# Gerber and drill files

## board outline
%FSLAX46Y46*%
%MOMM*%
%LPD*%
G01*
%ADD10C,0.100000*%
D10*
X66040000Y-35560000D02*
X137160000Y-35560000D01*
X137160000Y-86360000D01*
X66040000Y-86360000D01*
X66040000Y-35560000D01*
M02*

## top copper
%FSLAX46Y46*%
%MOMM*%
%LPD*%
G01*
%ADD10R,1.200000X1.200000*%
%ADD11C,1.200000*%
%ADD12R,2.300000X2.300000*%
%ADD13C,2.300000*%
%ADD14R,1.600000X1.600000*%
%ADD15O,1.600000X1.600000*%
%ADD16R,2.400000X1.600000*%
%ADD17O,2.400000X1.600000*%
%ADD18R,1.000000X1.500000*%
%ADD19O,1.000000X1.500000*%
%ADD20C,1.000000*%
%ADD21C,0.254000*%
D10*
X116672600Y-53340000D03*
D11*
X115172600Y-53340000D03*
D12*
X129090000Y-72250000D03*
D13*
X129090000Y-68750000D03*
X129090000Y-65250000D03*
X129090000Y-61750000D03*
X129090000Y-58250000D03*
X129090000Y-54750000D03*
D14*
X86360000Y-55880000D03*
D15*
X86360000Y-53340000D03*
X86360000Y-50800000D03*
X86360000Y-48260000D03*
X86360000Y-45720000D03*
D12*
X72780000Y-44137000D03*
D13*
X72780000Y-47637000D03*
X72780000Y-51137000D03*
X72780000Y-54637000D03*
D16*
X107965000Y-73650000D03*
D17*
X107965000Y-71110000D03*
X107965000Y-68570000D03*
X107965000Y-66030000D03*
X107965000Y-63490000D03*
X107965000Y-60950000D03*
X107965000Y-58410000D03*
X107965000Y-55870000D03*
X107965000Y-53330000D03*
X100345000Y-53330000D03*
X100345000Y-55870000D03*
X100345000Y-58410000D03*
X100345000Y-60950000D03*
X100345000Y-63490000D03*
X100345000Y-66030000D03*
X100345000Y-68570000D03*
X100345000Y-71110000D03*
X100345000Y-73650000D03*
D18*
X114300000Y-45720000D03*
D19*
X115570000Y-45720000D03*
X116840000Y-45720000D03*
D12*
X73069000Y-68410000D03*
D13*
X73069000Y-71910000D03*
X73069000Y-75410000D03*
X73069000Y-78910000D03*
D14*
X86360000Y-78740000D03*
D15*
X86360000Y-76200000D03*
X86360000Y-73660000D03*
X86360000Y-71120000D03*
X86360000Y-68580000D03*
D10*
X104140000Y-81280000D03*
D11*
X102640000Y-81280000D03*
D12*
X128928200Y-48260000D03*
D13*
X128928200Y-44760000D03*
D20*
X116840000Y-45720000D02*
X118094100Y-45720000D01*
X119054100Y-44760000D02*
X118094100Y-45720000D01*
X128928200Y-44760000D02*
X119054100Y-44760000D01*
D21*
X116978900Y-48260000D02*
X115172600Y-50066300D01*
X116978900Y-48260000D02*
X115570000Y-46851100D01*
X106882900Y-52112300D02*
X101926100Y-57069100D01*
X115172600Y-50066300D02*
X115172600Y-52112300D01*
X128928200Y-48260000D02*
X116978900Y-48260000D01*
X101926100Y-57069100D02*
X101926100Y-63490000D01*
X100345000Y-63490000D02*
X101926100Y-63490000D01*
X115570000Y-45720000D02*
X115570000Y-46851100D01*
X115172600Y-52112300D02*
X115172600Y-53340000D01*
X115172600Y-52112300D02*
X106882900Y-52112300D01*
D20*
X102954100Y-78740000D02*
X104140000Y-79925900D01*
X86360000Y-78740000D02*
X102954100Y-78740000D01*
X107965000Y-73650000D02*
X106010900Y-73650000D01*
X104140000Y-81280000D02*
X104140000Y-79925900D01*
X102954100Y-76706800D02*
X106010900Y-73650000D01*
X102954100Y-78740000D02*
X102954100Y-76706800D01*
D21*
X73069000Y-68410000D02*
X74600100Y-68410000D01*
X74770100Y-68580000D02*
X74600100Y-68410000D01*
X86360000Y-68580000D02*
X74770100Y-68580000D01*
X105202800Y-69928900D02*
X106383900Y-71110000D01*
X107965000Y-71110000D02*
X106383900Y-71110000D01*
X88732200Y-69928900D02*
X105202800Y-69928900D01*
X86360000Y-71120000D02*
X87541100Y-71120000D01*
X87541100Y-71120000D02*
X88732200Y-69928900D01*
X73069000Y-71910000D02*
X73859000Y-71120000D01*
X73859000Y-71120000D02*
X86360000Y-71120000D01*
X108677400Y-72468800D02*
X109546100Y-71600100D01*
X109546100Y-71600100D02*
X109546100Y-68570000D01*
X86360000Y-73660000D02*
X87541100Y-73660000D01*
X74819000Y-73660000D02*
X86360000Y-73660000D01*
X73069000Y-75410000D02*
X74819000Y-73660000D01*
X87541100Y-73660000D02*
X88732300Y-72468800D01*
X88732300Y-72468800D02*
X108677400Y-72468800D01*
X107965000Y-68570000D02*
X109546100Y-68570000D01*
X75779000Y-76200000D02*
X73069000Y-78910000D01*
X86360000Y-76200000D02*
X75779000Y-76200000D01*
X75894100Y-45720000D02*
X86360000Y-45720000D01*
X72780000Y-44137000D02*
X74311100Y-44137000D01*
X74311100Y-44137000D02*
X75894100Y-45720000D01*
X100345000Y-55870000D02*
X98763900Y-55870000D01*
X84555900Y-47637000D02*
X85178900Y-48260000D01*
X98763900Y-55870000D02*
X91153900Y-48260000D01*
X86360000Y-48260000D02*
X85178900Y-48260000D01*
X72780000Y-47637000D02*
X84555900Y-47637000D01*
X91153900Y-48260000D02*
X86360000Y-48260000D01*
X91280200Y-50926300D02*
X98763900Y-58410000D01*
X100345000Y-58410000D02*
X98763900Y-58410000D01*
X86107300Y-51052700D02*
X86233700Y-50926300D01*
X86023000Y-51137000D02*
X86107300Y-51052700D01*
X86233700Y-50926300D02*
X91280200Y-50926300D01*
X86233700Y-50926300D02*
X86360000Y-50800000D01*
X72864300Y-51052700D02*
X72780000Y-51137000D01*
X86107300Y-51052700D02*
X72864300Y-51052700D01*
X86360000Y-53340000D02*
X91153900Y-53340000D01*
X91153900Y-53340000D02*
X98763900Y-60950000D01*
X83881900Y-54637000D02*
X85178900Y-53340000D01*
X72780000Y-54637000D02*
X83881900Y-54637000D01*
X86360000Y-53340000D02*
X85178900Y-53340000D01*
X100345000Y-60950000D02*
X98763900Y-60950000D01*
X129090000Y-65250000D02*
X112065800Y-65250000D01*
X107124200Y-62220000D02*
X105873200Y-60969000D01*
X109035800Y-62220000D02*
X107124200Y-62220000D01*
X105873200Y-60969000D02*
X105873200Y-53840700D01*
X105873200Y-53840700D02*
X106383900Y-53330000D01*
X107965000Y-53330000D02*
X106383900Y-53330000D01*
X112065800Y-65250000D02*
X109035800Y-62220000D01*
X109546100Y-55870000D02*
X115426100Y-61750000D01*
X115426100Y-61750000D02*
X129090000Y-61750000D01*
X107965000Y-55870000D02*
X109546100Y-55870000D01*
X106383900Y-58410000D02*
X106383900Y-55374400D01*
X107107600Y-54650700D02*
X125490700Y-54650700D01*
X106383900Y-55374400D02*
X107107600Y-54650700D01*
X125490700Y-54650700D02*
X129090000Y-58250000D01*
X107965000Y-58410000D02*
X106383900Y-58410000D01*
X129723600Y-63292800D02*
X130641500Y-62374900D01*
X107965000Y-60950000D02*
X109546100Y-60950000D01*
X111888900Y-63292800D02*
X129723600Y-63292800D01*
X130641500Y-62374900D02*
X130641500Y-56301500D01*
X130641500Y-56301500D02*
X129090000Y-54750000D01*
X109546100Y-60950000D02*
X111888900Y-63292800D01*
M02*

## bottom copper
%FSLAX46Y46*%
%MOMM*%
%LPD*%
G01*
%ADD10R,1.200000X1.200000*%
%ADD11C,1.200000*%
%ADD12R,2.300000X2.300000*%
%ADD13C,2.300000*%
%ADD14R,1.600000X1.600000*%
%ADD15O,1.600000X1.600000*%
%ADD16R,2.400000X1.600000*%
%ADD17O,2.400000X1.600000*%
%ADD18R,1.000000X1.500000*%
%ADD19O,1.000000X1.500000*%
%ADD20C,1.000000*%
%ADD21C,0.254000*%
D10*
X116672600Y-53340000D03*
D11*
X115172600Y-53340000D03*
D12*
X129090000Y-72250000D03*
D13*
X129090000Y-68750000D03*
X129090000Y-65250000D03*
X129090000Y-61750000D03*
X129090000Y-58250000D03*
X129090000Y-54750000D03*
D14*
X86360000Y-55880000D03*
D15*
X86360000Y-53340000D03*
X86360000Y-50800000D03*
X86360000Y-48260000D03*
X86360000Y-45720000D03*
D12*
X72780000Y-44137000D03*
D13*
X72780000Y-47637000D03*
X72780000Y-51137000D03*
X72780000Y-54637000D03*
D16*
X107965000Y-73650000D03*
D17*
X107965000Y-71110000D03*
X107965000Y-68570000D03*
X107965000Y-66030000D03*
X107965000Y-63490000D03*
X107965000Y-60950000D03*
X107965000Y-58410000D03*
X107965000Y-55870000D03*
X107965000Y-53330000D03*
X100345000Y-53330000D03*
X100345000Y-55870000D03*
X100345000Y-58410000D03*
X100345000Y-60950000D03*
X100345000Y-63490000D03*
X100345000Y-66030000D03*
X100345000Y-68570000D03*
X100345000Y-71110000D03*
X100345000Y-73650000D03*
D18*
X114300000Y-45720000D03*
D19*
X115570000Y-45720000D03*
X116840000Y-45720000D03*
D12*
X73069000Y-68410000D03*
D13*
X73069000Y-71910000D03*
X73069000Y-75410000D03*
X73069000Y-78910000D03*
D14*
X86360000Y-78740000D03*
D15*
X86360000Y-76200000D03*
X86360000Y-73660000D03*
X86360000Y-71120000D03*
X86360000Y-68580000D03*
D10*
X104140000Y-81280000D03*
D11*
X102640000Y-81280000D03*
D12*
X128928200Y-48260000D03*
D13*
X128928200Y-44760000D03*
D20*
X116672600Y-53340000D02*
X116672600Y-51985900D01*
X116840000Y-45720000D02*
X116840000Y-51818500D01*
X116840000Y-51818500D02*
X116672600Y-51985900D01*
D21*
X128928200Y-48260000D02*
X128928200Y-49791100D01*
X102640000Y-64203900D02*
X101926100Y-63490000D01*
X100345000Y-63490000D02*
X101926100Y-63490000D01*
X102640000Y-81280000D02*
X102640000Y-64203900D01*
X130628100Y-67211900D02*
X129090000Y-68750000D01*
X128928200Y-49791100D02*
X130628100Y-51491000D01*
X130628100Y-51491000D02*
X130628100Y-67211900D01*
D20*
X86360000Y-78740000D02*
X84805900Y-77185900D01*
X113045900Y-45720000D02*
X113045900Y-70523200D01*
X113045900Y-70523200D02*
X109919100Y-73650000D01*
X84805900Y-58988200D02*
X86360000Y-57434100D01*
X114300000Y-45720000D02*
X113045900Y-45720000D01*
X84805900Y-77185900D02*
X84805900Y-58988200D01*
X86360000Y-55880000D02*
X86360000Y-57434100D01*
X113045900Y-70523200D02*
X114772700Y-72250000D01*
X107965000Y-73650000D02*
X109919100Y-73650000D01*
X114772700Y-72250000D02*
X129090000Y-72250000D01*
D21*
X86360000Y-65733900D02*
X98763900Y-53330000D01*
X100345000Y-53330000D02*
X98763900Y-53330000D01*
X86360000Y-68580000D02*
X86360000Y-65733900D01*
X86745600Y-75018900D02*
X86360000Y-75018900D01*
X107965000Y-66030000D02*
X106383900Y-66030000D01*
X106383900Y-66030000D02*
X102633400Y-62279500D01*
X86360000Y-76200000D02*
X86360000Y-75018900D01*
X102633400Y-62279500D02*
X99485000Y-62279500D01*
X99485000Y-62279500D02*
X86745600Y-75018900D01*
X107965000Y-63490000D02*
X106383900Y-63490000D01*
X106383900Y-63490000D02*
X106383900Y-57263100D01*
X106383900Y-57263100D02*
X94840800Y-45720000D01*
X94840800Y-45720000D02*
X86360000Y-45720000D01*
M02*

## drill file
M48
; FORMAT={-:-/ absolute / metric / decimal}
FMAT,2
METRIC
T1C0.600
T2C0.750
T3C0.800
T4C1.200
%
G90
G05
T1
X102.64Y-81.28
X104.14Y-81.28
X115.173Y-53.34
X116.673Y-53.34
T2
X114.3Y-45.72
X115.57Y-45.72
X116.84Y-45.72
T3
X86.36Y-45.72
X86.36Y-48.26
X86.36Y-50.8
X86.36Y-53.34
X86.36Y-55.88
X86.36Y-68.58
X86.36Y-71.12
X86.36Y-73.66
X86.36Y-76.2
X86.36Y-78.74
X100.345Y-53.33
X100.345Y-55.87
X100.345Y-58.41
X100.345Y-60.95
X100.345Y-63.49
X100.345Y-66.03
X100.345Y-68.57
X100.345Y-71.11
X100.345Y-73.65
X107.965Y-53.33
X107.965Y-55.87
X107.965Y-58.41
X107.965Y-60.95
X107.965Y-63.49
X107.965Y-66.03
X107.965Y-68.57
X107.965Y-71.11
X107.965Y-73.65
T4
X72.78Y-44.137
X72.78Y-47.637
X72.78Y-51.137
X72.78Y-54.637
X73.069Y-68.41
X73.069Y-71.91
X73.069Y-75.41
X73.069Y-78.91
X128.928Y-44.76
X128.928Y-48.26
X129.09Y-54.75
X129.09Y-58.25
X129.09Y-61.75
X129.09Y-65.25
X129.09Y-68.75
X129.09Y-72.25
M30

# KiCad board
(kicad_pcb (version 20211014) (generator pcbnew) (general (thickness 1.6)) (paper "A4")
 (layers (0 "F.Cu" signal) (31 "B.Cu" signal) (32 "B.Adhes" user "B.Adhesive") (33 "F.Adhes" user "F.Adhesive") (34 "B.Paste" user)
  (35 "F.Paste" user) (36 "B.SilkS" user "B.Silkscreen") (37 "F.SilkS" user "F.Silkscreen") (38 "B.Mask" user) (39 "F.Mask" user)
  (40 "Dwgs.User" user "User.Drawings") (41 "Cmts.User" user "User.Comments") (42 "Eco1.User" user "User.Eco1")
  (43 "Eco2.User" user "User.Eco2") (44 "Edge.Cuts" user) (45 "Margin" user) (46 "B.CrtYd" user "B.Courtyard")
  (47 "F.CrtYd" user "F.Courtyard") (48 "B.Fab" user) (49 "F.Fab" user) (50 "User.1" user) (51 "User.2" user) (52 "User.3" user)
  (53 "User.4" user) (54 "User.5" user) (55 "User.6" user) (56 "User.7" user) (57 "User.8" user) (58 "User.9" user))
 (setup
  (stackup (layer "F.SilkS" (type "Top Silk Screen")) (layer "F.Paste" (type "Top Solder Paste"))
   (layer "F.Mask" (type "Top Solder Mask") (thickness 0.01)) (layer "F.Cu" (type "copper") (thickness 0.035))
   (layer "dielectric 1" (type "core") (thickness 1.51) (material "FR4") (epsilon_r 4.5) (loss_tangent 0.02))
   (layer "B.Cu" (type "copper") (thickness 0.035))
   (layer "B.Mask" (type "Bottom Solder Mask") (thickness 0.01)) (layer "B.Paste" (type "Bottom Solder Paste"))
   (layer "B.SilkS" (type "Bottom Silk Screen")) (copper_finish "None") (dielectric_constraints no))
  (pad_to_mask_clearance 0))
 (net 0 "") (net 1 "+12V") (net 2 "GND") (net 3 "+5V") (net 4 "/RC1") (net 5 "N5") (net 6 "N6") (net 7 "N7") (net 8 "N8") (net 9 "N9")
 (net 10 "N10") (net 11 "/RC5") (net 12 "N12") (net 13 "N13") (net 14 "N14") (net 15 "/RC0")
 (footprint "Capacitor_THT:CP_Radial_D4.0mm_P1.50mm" (layer "F.Cu") (at 116.6726 53.34 180)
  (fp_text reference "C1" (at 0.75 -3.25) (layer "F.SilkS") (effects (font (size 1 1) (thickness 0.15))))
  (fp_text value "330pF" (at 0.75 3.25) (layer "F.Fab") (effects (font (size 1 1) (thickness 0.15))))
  (pad "1" thru_hole rect (at 0 0 180) (size 1.2 1.2) (drill 0.6) (layers *.Cu *.Mask) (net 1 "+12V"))
  (pad "2" thru_hole circle (at 1.5 0 180) (size 1.2 1.2) (drill 0.6) (layers *.Cu *.Mask) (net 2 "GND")))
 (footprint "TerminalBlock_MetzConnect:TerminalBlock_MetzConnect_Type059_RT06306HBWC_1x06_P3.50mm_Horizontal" (layer "F.Cu")
  (at 129.09 72.25 90)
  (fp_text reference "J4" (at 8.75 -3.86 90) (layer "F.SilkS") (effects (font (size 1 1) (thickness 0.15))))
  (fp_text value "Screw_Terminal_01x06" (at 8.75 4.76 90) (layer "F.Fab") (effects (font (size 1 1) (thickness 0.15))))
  (pad "1" thru_hole rect (at 0 0 90) (size 2.3 2.3) (drill 1.2) (layers *.Cu *.Mask) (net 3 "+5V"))
  (pad "2" thru_hole circle (at 3.5 0 90) (size 2.3 2.3) (drill 1.2) (layers *.Cu *.Mask) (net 2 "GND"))
  (pad "3" thru_hole circle (at 7 0 90) (size 2.3 2.3) (drill 1.2) (layers *.Cu *.Mask) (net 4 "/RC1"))
  (pad "4" thru_hole circle (at 10.5 0 90) (size 2.3 2.3) (drill 1.2) (layers *.Cu *.Mask) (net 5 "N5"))
  (pad "5" thru_hole circle (at 14 0 90) (size 2.3 2.3) (drill 1.2) (layers *.Cu *.Mask) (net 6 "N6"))
  (pad "6" thru_hole circle (at 17.5 0 90) (size 2.3 2.3) (drill 1.2) (layers *.Cu *.Mask) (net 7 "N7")))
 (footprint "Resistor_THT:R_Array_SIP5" (layer "F.Cu") (at 86.36 55.88 90)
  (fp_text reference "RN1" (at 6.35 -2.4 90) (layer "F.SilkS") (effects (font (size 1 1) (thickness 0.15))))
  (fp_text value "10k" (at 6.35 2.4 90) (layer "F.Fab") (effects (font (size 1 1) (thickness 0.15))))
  (pad "1" thru_hole rect (at 0 0 90) (size 1.6 1.6) (drill 0.8) (layers *.Cu *.Mask) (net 3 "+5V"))
  (pad "2" thru_hole oval (at 2.54 0 90) (size 1.6 1.6) (drill 0.8) (layers *.Cu *.Mask) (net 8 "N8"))
  (pad "3" thru_hole oval (at 5.08 0 90) (size 1.6 1.6) (drill 0.8) (layers *.Cu *.Mask) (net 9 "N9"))
  (pad "4" thru_hole oval (at 7.62 0 90) (size 1.6 1.6) (drill 0.8) (layers *.Cu *.Mask) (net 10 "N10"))
  (pad "5" thru_hole oval (at 10.16 0 90) (size 1.6 1.6) (drill 0.8) (layers *.Cu *.Mask) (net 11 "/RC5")))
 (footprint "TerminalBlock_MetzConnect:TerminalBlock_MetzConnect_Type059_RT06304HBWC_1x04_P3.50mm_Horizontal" (layer "F.Cu")
  (at 72.78 44.137 -90)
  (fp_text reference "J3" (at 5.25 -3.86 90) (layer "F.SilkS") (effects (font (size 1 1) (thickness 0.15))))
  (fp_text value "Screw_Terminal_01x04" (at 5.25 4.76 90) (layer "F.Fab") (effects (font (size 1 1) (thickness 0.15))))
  (pad "1" thru_hole rect (at 0 0 270) (size 2.3 2.3) (drill 1.2) (layers *.Cu *.Mask) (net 11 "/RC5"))
  (pad "2" thru_hole circle (at 3.5 0 270) (size 2.3 2.3) (drill 1.2) (layers *.Cu *.Mask) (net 10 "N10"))
  (pad "3" thru_hole circle (at 7 0 270) (size 2.3 2.3) (drill 1.2) (layers *.Cu *.Mask) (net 9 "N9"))
  (pad "4" thru_hole circle (at 10.5 0 270) (size 2.3 2.3) (drill 1.2) (layers *.Cu *.Mask) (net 8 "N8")))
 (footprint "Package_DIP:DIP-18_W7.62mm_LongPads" (layer "F.Cu") (at 107.965 73.65 180)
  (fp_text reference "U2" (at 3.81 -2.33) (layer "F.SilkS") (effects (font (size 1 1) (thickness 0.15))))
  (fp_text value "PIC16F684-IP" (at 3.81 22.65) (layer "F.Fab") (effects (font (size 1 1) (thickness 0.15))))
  (pad "1" thru_hole rect (at 0 0 180) (size 2.4 1.6) (drill 0.8) (layers *.Cu *.Mask) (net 3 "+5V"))
  (pad "2" thru_hole oval (at 0 2.54 180) (size 2.4 1.6) (drill 0.8) (layers *.Cu *.Mask) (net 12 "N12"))
  (pad "3" thru_hole oval (at 0 5.08 180) (size 2.4 1.6) (drill 0.8) (layers *.Cu *.Mask) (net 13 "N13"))
  (pad "4" thru_hole oval (at 0 7.62 180) (size 2.4 1.6) (drill 0.8) (layers *.Cu *.Mask) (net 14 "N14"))
  (pad "5" thru_hole oval (at 0 10.16 180) (size 2.4 1.6) (drill 0.8) (layers *.Cu *.Mask) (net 11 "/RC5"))
  (pad "6" thru_hole oval (at 0 12.7 180) (size 2.4 1.6) (drill 0.8) (layers *.Cu *.Mask) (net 7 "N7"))
  (pad "7" thru_hole oval (at 0 15.24 180) (size 2.4 1.6) (drill 0.8) (layers *.Cu *.Mask) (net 6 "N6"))
  (pad "8" thru_hole oval (at 0 17.78 180) (size 2.4 1.6) (drill 0.8) (layers *.Cu *.Mask) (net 5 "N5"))
  (pad "9" thru_hole oval (at 0 20.32 180) (size 2.4 1.6) (drill 0.8) (layers *.Cu *.Mask) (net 4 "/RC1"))
  (pad "10" thru_hole oval (at 7.62 20.32 180) (size 2.4 1.6) (drill 0.8) (layers *.Cu *.Mask) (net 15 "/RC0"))
  (pad "11" thru_hole oval (at 7.62 17.78 180) (size 2.4 1.6) (drill 0.8) (layers *.Cu *.Mask) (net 10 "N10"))
  (pad "12" thru_hole oval (at 7.62 15.24 180) (size 2.4 1.6) (drill 0.8) (layers *.Cu *.Mask) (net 9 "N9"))
  (pad "13" thru_hole oval (at 7.62 12.7 180) (size 2.4 1.6) (drill 0.8) (layers *.Cu *.Mask) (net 8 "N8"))
  (pad "14" thru_hole oval (at 7.62 10.16 180) (size 2.4 1.6) (drill 0.8) (layers *.Cu *.Mask) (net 2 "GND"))
  (pad "15" thru_hole oval (at 7.62 7.62 180) (size 2.4 1.6) (drill 0.8) (layers *.Cu *.Mask))
  (pad "16" thru_hole oval (at 7.62 5.08 180) (size 2.4 1.6) (drill 0.8) (layers *.Cu *.Mask))
  (pad "17" thru_hole oval (at 7.62 2.54 180) (size 2.4 1.6) (drill 0.8) (layers *.Cu *.Mask))
  (pad "18" thru_hole oval (at 7.62 0 180) (size 2.4 1.6) (drill 0.8) (layers *.Cu *.Mask)))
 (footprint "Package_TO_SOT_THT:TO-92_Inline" (layer "F.Cu") (at 114.3 45.72)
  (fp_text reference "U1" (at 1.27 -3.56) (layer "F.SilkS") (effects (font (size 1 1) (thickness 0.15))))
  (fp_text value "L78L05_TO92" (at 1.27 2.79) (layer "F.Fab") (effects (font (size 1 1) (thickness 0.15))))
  (pad "1" thru_hole rect (at 0 0) (size 1 1.5) (drill 0.75) (layers *.Cu *.Mask) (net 3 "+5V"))
  (pad "2" thru_hole oval (at 1.27 0) (size 1 1.5) (drill 0.75) (layers *.Cu *.Mask) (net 2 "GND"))
  (pad "3" thru_hole oval (at 2.54 0) (size 1 1.5) (drill 0.75) (layers *.Cu *.Mask) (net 1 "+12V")))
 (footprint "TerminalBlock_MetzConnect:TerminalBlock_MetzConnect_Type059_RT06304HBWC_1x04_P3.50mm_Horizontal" (layer "F.Cu")
  (at 73.069 68.41 -90)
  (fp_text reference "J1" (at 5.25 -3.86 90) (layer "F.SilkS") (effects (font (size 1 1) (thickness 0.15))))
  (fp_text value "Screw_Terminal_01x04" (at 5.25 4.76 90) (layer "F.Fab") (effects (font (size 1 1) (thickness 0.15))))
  (pad "1" thru_hole rect (at 0 0 270) (size 2.3 2.3) (drill 1.2) (layers *.Cu *.Mask) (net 15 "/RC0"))
  (pad "2" thru_hole circle (at 3.5 0 270) (size 2.3 2.3) (drill 1.2) (layers *.Cu *.Mask) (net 12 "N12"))
  (pad "3" thru_hole circle (at 7 0 270) (size 2.3 2.3) (drill 1.2) (layers *.Cu *.Mask) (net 13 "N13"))
  (pad "4" thru_hole circle (at 10.5 0 270) (size 2.3 2.3) (drill 1.2) (layers *.Cu *.Mask) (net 14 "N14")))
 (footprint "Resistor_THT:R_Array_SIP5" (layer "F.Cu") (at 86.36 78.74 90)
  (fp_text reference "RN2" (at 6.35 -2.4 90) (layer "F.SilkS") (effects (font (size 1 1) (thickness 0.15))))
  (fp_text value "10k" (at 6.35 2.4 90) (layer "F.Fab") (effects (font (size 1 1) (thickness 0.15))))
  (pad "1" thru_hole rect (at 0 0 90) (size 1.6 1.6) (drill 0.8) (layers *.Cu *.Mask) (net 3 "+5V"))
  (pad "2" thru_hole oval (at 2.54 0 90) (size 1.6 1.6) (drill 0.8) (layers *.Cu *.Mask) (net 14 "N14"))
  (pad "3" thru_hole oval (at 5.08 0 90) (size 1.6 1.6) (drill 0.8) (layers *.Cu *.Mask) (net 13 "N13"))
  (pad "4" thru_hole oval (at 7.62 0 90) (size 1.6 1.6) (drill 0.8) (layers *.Cu *.Mask) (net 12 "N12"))
  (pad "5" thru_hole oval (at 10.16 0 90) (size 1.6 1.6) (drill 0.8) (layers *.Cu *.Mask) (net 15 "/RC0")))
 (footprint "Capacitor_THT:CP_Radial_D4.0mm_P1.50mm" (layer "F.Cu") (at 104.14 81.28 180)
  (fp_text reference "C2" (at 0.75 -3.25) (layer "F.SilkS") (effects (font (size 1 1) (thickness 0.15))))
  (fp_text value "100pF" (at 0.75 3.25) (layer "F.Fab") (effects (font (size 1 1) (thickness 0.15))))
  (pad "1" thru_hole rect (at 0 0 180) (size 1.2 1.2) (drill 0.6) (layers *.Cu *.Mask) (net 3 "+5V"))
  (pad "2" thru_hole circle (at 1.5 0 180) (size 1.2 1.2) (drill 0.6) (layers *.Cu *.Mask) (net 2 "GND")))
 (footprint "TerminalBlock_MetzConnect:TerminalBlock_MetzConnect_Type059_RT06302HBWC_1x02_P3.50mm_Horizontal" (layer "F.Cu")
  (at 128.9282 48.26 90)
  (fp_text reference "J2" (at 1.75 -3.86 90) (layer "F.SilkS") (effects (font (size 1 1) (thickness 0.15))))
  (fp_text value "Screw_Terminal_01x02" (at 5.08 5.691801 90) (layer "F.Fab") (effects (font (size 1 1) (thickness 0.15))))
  (pad "1" thru_hole rect (at 0 0 90) (size 2.3 2.3) (drill 1.2) (layers *.Cu *.Mask) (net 2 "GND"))
  (pad "2" thru_hole circle (at 3.5 0 90) (size 2.3 2.3) (drill 1.2) (layers *.Cu *.Mask) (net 1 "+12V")))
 (gr_rect (start 66.04 35.56) (end 137.16 86.36) (layer "Edge.Cuts") (width 0.1) (fill none))
 (segment (start 116.84 45.72) (end 118.0941 45.72) (width 1) (layer "F.Cu") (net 1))
 (segment (start 119.0541 44.76) (end 118.0941 45.72) (width 1) (layer "F.Cu") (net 1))
 (segment (start 128.9282 44.76) (end 119.0541 44.76) (width 1) (layer "F.Cu") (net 1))
 (segment (start 116.6726 53.34) (end 116.6726 51.9859) (width 1) (layer "B.Cu") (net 1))
 (segment (start 116.84 45.72) (end 116.84 51.8185) (width 1) (layer "B.Cu") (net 1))
 (segment (start 116.84 51.8185) (end 116.6726 51.9859) (width 1) (layer "B.Cu") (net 1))
 (segment (start 116.9789 48.26) (end 115.1726 50.0663) (width 0.254) (layer "F.Cu") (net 2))
 (segment (start 116.9789 48.26) (end 115.57 46.8511) (width 0.254) (layer "F.Cu") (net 2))
 (segment (start 106.8829 52.1123) (end 101.9261 57.0691) (width 0.254) (layer "F.Cu") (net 2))
 (segment (start 115.1726 50.0663) (end 115.1726 52.1123) (width 0.254) (layer "F.Cu") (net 2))
 (segment (start 128.9282 48.26) (end 116.9789 48.26) (width 0.254) (layer "F.Cu") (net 2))
 (segment (start 101.9261 57.0691) (end 101.9261 63.49) (width 0.254) (layer "F.Cu") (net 2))
 (segment (start 100.345 63.49) (end 101.9261 63.49) (width 0.254) (layer "F.Cu") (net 2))
 (segment (start 115.57 45.72) (end 115.57 46.8511) (width 0.254) (layer "F.Cu") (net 2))
 (segment (start 115.1726 52.1123) (end 115.1726 53.34) (width 0.254) (layer "F.Cu") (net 2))
 (segment (start 115.1726 52.1123) (end 106.8829 52.1123) (width 0.254) (layer "F.Cu") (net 2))
 (segment (start 128.9282 48.26) (end 128.9282 49.7911) (width 0.254) (layer "B.Cu") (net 2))
 (segment (start 102.64 64.2039) (end 101.9261 63.49) (width 0.254) (layer "B.Cu") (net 2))
 (segment (start 100.345 63.49) (end 101.9261 63.49) (width 0.254) (layer "B.Cu") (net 2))
 (segment (start 102.64 81.28) (end 102.64 64.2039) (width 0.254) (layer "B.Cu") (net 2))
 (segment (start 130.6281 67.2119) (end 129.09 68.75) (width 0.254) (layer "B.Cu") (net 2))
 (segment (start 128.9282 49.7911) (end 130.6281 51.491) (width 0.254) (layer "B.Cu") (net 2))
 (segment (start 130.6281 51.491) (end 130.6281 67.2119) (width 0.254) (layer "B.Cu") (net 2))
 (segment (start 102.9541 78.74) (end 104.14 79.9259) (width 1) (layer "F.Cu") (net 3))
 (segment (start 86.36 78.74) (end 102.9541 78.74) (width 1) (layer "F.Cu") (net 3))
 (segment (start 107.965 73.65) (end 106.0109 73.65) (width 1) (layer "F.Cu") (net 3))
 (segment (start 104.14 81.28) (end 104.14 79.9259) (width 1) (layer "F.Cu") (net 3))
 (segment (start 102.9541 76.7068) (end 106.0109 73.65) (width 1) (layer "F.Cu") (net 3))
 (segment (start 102.9541 78.74) (end 102.9541 76.7068) (width 1) (layer "F.Cu") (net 3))
 (segment (start 86.36 78.74) (end 84.8059 77.1859) (width 1) (layer "B.Cu") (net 3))
 (segment (start 113.0459 45.72) (end 113.0459 70.5232) (width 1) (layer "B.Cu") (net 3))
 (segment (start 113.0459 70.5232) (end 109.9191 73.65) (width 1) (layer "B.Cu") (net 3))
 (segment (start 84.8059 58.9882) (end 86.36 57.4341) (width 1) (layer "B.Cu") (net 3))
 (segment (start 114.3 45.72) (end 113.0459 45.72) (width 1) (layer "B.Cu") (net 3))
 (segment (start 84.8059 77.1859) (end 84.8059 58.9882) (width 1) (layer "B.Cu") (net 3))
 (segment (start 86.36 55.88) (end 86.36 57.4341) (width 1) (layer "B.Cu") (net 3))
 (segment (start 113.0459 70.5232) (end 114.7727 72.25) (width 1) (layer "B.Cu") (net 3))
 (segment (start 107.965 73.65) (end 109.9191 73.65) (width 1) (layer "B.Cu") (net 3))
 (segment (start 114.7727 72.25) (end 129.09 72.25) (width 1) (layer "B.Cu") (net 3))
 (segment (start 73.069 68.41) (end 74.6001 68.41) (width 0.254) (layer "F.Cu") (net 15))
 (segment (start 74.7701 68.58) (end 74.6001 68.41) (width 0.254) (layer "F.Cu") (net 15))
 (segment (start 86.36 68.58) (end 74.7701 68.58) (width 0.254) (layer "F.Cu") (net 15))
 (segment (start 86.36 65.7339) (end 98.7639 53.33) (width 0.254) (layer "B.Cu") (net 15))
 (segment (start 100.345 53.33) (end 98.7639 53.33) (width 0.254) (layer "B.Cu") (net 15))
 (segment (start 86.36 68.58) (end 86.36 65.7339) (width 0.254) (layer "B.Cu") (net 15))
 (segment (start 105.2028 69.9289) (end 106.3839 71.11) (width 0.254) (layer "F.Cu") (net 12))
 (segment (start 107.965 71.11) (end 106.3839 71.11) (width 0.254) (layer "F.Cu") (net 12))
 (segment (start 88.7322 69.9289) (end 105.2028 69.9289) (width 0.254) (layer "F.Cu") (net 12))
 (segment (start 86.36 71.12) (end 87.5411 71.12) (width 0.254) (layer "F.Cu") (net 12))
 (segment (start 87.5411 71.12) (end 88.7322 69.9289) (width 0.254) (layer "F.Cu") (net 12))
 (segment (start 73.069 71.91) (end 73.859 71.12) (width 0.254) (layer "F.Cu") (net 12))
 (segment (start 73.859 71.12) (end 86.36 71.12) (width 0.254) (layer "F.Cu") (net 12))
 (segment (start 108.6774 72.4688) (end 109.5461 71.6001) (width 0.254) (layer "F.Cu") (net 13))
 (segment (start 109.5461 71.6001) (end 109.5461 68.57) (width 0.254) (layer "F.Cu") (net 13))
 (segment (start 86.36 73.66) (end 87.5411 73.66) (width 0.254) (layer "F.Cu") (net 13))
 (segment (start 74.819 73.66) (end 86.36 73.66) (width 0.254) (layer "F.Cu") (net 13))
 (segment (start 73.069 75.41) (end 74.819 73.66) (width 0.254) (layer "F.Cu") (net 13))
 (segment (start 87.5411 73.66) (end 88.7323 72.4688) (width 0.254) (layer "F.Cu") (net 13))
 (segment (start 88.7323 72.4688) (end 108.6774 72.4688) (width 0.254) (layer "F.Cu") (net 13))
 (segment (start 107.965 68.57) (end 109.5461 68.57) (width 0.254) (layer "F.Cu") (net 13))
 (segment (start 75.779 76.2) (end 73.069 78.91) (width 0.254) (layer "F.Cu") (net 14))
 (segment (start 86.36 76.2) (end 75.779 76.2) (width 0.254) (layer "F.Cu") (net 14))
 (segment (start 86.7456 75.0189) (end 86.36 75.0189) (width 0.254) (layer "B.Cu") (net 14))
 (segment (start 107.965 66.03) (end 106.3839 66.03) (width 0.254) (layer "B.Cu") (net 14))
 (segment (start 106.3839 66.03) (end 102.6334 62.2795) (width 0.254) (layer "B.Cu") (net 14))
 (segment (start 86.36 76.2) (end 86.36 75.0189) (width 0.254) (layer "B.Cu") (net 14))
 (segment (start 102.6334 62.2795) (end 99.485 62.2795) (width 0.254) (layer "B.Cu") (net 14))
 (segment (start 99.485 62.2795) (end 86.7456 75.0189) (width 0.254) (layer "B.Cu") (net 14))
 (segment (start 75.8941 45.72) (end 86.36 45.72) (width 0.254) (layer "F.Cu") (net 11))
 (segment (start 72.78 44.137) (end 74.3111 44.137) (width 0.254) (layer "F.Cu") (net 11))
 (segment (start 74.3111 44.137) (end 75.8941 45.72) (width 0.254) (layer "F.Cu") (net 11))
 (segment (start 107.965 63.49) (end 106.3839 63.49) (width 0.254) (layer "B.Cu") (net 11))
 (segment (start 106.3839 63.49) (end 106.3839 57.2631) (width 0.254) (layer "B.Cu") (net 11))
 (segment (start 106.3839 57.2631) (end 94.8408 45.72) (width 0.254) (layer "B.Cu") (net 11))
 (segment (start 94.8408 45.72) (end 86.36 45.72) (width 0.254) (layer "B.Cu") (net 11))
 (segment (start 100.345 55.87) (end 98.7639 55.87) (width 0.254) (layer "F.Cu") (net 10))
 (segment (start 84.5559 47.637) (end 85.1789 48.26) (width 0.254) (layer "F.Cu") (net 10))
 (segment (start 98.7639 55.87) (end 91.1539 48.26) (width 0.254) (layer "F.Cu") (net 10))
 (segment (start 86.36 48.26) (end 85.1789 48.26) (width 0.254) (layer "F.Cu") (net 10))
 (segment (start 72.78 47.637) (end 84.5559 47.637) (width 0.254) (layer "F.Cu") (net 10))
 (segment (start 91.1539 48.26) (end 86.36 48.26) (width 0.254) (layer "F.Cu") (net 10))
 (segment (start 91.2802 50.9263) (end 98.7639 58.41) (width 0.254) (layer "F.Cu") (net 9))
 (segment (start 100.345 58.41) (end 98.7639 58.41) (width 0.254) (layer "F.Cu") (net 9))
 (segment (start 86.1073 51.0527) (end 86.2337 50.9263) (width 0.254) (layer "F.Cu") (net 9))
 (segment (start 86.023 51.137) (end 86.1073 51.0527) (width 0.254) (layer "F.Cu") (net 9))
 (segment (start 86.2337 50.9263) (end 91.2802 50.9263) (width 0.254) (layer "F.Cu") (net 9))
 (segment (start 86.2337 50.9263) (end 86.36 50.8) (width 0.254) (layer "F.Cu") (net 9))
 (segment (start 72.8643 51.0527) (end 72.78 51.137) (width 0.254) (layer "F.Cu") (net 9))
 (segment (start 86.1073 51.0527) (end 72.8643 51.0527) (width 0.254) (layer "F.Cu") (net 9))
 (segment (start 86.36 53.34) (end 91.1539 53.34) (width 0.254) (layer "F.Cu") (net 8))
 (segment (start 91.1539 53.34) (end 98.7639 60.95) (width 0.254) (layer "F.Cu") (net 8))
 (segment (start 83.8819 54.637) (end 85.1789 53.34) (width 0.254) (layer "F.Cu") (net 8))
 (segment (start 72.78 54.637) (end 83.8819 54.637) (width 0.254) (layer "F.Cu") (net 8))
 (segment (start 86.36 53.34) (end 85.1789 53.34) (width 0.254) (layer "F.Cu") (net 8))
 (segment (start 100.345 60.95) (end 98.7639 60.95) (width 0.254) (layer "F.Cu") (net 8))
 (segment (start 129.09 65.25) (end 112.0658 65.25) (width 0.254) (layer "F.Cu") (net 4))
 (segment (start 107.1242 62.22) (end 105.8732 60.969) (width 0.254) (layer "F.Cu") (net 4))
 (segment (start 109.0358 62.22) (end 107.1242 62.22) (width 0.254) (layer "F.Cu") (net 4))
 (segment (start 105.8732 60.969) (end 105.8732 53.8407) (width 0.254) (layer "F.Cu") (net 4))
 (segment (start 105.8732 53.8407) (end 106.3839 53.33) (width 0.254) (layer "F.Cu") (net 4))
 (segment (start 107.965 53.33) (end 106.3839 53.33) (width 0.254) (layer "F.Cu") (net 4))
 (segment (start 112.0658 65.25) (end 109.0358 62.22) (width 0.254) (layer "F.Cu") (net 4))
 (segment (start 109.5461 55.87) (end 115.4261 61.75) (width 0.254) (layer "F.Cu") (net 5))
 (segment (start 115.4261 61.75) (end 129.09 61.75) (width 0.254) (layer "F.Cu") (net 5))
 (segment (start 107.965 55.87) (end 109.5461 55.87) (width 0.254) (layer "F.Cu") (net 5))
 (segment (start 106.3839 58.41) (end 106.3839 55.3744) (width 0.254) (layer "F.Cu") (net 6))
 (segment (start 107.1076 54.6507) (end 125.4907 54.6507) (width 0.254) (layer "F.Cu") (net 6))
 (segment (start 106.3839 55.3744) (end 107.1076 54.6507) (width 0.254) (layer "F.Cu") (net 6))
 (segment (start 125.4907 54.6507) (end 129.09 58.25) (width 0.254) (layer "F.Cu") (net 6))
 (segment (start 107.965 58.41) (end 106.3839 58.41) (width 0.254) (layer "F.Cu") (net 6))
 (segment (start 129.7236 63.2928) (end 130.6415 62.3749) (width 0.254) (layer "F.Cu") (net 7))
 (segment (start 107.965 60.95) (end 109.5461 60.95) (width 0.254) (layer "F.Cu") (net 7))
 (segment (start 111.8889 63.2928) (end 129.7236 63.2928) (width 0.254) (layer "F.Cu") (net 7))
 (segment (start 130.6415 62.3749) (end 130.6415 56.3015) (width 0.254) (layer "F.Cu") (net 7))
 (segment (start 130.6415 56.3015) (end 129.09 54.75) (width 0.254) (layer "F.Cu") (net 7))
 (segment (start 109.5461 60.95) (end 111.8889 63.2928) (width 0.254) (layer "F.Cu") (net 7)))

